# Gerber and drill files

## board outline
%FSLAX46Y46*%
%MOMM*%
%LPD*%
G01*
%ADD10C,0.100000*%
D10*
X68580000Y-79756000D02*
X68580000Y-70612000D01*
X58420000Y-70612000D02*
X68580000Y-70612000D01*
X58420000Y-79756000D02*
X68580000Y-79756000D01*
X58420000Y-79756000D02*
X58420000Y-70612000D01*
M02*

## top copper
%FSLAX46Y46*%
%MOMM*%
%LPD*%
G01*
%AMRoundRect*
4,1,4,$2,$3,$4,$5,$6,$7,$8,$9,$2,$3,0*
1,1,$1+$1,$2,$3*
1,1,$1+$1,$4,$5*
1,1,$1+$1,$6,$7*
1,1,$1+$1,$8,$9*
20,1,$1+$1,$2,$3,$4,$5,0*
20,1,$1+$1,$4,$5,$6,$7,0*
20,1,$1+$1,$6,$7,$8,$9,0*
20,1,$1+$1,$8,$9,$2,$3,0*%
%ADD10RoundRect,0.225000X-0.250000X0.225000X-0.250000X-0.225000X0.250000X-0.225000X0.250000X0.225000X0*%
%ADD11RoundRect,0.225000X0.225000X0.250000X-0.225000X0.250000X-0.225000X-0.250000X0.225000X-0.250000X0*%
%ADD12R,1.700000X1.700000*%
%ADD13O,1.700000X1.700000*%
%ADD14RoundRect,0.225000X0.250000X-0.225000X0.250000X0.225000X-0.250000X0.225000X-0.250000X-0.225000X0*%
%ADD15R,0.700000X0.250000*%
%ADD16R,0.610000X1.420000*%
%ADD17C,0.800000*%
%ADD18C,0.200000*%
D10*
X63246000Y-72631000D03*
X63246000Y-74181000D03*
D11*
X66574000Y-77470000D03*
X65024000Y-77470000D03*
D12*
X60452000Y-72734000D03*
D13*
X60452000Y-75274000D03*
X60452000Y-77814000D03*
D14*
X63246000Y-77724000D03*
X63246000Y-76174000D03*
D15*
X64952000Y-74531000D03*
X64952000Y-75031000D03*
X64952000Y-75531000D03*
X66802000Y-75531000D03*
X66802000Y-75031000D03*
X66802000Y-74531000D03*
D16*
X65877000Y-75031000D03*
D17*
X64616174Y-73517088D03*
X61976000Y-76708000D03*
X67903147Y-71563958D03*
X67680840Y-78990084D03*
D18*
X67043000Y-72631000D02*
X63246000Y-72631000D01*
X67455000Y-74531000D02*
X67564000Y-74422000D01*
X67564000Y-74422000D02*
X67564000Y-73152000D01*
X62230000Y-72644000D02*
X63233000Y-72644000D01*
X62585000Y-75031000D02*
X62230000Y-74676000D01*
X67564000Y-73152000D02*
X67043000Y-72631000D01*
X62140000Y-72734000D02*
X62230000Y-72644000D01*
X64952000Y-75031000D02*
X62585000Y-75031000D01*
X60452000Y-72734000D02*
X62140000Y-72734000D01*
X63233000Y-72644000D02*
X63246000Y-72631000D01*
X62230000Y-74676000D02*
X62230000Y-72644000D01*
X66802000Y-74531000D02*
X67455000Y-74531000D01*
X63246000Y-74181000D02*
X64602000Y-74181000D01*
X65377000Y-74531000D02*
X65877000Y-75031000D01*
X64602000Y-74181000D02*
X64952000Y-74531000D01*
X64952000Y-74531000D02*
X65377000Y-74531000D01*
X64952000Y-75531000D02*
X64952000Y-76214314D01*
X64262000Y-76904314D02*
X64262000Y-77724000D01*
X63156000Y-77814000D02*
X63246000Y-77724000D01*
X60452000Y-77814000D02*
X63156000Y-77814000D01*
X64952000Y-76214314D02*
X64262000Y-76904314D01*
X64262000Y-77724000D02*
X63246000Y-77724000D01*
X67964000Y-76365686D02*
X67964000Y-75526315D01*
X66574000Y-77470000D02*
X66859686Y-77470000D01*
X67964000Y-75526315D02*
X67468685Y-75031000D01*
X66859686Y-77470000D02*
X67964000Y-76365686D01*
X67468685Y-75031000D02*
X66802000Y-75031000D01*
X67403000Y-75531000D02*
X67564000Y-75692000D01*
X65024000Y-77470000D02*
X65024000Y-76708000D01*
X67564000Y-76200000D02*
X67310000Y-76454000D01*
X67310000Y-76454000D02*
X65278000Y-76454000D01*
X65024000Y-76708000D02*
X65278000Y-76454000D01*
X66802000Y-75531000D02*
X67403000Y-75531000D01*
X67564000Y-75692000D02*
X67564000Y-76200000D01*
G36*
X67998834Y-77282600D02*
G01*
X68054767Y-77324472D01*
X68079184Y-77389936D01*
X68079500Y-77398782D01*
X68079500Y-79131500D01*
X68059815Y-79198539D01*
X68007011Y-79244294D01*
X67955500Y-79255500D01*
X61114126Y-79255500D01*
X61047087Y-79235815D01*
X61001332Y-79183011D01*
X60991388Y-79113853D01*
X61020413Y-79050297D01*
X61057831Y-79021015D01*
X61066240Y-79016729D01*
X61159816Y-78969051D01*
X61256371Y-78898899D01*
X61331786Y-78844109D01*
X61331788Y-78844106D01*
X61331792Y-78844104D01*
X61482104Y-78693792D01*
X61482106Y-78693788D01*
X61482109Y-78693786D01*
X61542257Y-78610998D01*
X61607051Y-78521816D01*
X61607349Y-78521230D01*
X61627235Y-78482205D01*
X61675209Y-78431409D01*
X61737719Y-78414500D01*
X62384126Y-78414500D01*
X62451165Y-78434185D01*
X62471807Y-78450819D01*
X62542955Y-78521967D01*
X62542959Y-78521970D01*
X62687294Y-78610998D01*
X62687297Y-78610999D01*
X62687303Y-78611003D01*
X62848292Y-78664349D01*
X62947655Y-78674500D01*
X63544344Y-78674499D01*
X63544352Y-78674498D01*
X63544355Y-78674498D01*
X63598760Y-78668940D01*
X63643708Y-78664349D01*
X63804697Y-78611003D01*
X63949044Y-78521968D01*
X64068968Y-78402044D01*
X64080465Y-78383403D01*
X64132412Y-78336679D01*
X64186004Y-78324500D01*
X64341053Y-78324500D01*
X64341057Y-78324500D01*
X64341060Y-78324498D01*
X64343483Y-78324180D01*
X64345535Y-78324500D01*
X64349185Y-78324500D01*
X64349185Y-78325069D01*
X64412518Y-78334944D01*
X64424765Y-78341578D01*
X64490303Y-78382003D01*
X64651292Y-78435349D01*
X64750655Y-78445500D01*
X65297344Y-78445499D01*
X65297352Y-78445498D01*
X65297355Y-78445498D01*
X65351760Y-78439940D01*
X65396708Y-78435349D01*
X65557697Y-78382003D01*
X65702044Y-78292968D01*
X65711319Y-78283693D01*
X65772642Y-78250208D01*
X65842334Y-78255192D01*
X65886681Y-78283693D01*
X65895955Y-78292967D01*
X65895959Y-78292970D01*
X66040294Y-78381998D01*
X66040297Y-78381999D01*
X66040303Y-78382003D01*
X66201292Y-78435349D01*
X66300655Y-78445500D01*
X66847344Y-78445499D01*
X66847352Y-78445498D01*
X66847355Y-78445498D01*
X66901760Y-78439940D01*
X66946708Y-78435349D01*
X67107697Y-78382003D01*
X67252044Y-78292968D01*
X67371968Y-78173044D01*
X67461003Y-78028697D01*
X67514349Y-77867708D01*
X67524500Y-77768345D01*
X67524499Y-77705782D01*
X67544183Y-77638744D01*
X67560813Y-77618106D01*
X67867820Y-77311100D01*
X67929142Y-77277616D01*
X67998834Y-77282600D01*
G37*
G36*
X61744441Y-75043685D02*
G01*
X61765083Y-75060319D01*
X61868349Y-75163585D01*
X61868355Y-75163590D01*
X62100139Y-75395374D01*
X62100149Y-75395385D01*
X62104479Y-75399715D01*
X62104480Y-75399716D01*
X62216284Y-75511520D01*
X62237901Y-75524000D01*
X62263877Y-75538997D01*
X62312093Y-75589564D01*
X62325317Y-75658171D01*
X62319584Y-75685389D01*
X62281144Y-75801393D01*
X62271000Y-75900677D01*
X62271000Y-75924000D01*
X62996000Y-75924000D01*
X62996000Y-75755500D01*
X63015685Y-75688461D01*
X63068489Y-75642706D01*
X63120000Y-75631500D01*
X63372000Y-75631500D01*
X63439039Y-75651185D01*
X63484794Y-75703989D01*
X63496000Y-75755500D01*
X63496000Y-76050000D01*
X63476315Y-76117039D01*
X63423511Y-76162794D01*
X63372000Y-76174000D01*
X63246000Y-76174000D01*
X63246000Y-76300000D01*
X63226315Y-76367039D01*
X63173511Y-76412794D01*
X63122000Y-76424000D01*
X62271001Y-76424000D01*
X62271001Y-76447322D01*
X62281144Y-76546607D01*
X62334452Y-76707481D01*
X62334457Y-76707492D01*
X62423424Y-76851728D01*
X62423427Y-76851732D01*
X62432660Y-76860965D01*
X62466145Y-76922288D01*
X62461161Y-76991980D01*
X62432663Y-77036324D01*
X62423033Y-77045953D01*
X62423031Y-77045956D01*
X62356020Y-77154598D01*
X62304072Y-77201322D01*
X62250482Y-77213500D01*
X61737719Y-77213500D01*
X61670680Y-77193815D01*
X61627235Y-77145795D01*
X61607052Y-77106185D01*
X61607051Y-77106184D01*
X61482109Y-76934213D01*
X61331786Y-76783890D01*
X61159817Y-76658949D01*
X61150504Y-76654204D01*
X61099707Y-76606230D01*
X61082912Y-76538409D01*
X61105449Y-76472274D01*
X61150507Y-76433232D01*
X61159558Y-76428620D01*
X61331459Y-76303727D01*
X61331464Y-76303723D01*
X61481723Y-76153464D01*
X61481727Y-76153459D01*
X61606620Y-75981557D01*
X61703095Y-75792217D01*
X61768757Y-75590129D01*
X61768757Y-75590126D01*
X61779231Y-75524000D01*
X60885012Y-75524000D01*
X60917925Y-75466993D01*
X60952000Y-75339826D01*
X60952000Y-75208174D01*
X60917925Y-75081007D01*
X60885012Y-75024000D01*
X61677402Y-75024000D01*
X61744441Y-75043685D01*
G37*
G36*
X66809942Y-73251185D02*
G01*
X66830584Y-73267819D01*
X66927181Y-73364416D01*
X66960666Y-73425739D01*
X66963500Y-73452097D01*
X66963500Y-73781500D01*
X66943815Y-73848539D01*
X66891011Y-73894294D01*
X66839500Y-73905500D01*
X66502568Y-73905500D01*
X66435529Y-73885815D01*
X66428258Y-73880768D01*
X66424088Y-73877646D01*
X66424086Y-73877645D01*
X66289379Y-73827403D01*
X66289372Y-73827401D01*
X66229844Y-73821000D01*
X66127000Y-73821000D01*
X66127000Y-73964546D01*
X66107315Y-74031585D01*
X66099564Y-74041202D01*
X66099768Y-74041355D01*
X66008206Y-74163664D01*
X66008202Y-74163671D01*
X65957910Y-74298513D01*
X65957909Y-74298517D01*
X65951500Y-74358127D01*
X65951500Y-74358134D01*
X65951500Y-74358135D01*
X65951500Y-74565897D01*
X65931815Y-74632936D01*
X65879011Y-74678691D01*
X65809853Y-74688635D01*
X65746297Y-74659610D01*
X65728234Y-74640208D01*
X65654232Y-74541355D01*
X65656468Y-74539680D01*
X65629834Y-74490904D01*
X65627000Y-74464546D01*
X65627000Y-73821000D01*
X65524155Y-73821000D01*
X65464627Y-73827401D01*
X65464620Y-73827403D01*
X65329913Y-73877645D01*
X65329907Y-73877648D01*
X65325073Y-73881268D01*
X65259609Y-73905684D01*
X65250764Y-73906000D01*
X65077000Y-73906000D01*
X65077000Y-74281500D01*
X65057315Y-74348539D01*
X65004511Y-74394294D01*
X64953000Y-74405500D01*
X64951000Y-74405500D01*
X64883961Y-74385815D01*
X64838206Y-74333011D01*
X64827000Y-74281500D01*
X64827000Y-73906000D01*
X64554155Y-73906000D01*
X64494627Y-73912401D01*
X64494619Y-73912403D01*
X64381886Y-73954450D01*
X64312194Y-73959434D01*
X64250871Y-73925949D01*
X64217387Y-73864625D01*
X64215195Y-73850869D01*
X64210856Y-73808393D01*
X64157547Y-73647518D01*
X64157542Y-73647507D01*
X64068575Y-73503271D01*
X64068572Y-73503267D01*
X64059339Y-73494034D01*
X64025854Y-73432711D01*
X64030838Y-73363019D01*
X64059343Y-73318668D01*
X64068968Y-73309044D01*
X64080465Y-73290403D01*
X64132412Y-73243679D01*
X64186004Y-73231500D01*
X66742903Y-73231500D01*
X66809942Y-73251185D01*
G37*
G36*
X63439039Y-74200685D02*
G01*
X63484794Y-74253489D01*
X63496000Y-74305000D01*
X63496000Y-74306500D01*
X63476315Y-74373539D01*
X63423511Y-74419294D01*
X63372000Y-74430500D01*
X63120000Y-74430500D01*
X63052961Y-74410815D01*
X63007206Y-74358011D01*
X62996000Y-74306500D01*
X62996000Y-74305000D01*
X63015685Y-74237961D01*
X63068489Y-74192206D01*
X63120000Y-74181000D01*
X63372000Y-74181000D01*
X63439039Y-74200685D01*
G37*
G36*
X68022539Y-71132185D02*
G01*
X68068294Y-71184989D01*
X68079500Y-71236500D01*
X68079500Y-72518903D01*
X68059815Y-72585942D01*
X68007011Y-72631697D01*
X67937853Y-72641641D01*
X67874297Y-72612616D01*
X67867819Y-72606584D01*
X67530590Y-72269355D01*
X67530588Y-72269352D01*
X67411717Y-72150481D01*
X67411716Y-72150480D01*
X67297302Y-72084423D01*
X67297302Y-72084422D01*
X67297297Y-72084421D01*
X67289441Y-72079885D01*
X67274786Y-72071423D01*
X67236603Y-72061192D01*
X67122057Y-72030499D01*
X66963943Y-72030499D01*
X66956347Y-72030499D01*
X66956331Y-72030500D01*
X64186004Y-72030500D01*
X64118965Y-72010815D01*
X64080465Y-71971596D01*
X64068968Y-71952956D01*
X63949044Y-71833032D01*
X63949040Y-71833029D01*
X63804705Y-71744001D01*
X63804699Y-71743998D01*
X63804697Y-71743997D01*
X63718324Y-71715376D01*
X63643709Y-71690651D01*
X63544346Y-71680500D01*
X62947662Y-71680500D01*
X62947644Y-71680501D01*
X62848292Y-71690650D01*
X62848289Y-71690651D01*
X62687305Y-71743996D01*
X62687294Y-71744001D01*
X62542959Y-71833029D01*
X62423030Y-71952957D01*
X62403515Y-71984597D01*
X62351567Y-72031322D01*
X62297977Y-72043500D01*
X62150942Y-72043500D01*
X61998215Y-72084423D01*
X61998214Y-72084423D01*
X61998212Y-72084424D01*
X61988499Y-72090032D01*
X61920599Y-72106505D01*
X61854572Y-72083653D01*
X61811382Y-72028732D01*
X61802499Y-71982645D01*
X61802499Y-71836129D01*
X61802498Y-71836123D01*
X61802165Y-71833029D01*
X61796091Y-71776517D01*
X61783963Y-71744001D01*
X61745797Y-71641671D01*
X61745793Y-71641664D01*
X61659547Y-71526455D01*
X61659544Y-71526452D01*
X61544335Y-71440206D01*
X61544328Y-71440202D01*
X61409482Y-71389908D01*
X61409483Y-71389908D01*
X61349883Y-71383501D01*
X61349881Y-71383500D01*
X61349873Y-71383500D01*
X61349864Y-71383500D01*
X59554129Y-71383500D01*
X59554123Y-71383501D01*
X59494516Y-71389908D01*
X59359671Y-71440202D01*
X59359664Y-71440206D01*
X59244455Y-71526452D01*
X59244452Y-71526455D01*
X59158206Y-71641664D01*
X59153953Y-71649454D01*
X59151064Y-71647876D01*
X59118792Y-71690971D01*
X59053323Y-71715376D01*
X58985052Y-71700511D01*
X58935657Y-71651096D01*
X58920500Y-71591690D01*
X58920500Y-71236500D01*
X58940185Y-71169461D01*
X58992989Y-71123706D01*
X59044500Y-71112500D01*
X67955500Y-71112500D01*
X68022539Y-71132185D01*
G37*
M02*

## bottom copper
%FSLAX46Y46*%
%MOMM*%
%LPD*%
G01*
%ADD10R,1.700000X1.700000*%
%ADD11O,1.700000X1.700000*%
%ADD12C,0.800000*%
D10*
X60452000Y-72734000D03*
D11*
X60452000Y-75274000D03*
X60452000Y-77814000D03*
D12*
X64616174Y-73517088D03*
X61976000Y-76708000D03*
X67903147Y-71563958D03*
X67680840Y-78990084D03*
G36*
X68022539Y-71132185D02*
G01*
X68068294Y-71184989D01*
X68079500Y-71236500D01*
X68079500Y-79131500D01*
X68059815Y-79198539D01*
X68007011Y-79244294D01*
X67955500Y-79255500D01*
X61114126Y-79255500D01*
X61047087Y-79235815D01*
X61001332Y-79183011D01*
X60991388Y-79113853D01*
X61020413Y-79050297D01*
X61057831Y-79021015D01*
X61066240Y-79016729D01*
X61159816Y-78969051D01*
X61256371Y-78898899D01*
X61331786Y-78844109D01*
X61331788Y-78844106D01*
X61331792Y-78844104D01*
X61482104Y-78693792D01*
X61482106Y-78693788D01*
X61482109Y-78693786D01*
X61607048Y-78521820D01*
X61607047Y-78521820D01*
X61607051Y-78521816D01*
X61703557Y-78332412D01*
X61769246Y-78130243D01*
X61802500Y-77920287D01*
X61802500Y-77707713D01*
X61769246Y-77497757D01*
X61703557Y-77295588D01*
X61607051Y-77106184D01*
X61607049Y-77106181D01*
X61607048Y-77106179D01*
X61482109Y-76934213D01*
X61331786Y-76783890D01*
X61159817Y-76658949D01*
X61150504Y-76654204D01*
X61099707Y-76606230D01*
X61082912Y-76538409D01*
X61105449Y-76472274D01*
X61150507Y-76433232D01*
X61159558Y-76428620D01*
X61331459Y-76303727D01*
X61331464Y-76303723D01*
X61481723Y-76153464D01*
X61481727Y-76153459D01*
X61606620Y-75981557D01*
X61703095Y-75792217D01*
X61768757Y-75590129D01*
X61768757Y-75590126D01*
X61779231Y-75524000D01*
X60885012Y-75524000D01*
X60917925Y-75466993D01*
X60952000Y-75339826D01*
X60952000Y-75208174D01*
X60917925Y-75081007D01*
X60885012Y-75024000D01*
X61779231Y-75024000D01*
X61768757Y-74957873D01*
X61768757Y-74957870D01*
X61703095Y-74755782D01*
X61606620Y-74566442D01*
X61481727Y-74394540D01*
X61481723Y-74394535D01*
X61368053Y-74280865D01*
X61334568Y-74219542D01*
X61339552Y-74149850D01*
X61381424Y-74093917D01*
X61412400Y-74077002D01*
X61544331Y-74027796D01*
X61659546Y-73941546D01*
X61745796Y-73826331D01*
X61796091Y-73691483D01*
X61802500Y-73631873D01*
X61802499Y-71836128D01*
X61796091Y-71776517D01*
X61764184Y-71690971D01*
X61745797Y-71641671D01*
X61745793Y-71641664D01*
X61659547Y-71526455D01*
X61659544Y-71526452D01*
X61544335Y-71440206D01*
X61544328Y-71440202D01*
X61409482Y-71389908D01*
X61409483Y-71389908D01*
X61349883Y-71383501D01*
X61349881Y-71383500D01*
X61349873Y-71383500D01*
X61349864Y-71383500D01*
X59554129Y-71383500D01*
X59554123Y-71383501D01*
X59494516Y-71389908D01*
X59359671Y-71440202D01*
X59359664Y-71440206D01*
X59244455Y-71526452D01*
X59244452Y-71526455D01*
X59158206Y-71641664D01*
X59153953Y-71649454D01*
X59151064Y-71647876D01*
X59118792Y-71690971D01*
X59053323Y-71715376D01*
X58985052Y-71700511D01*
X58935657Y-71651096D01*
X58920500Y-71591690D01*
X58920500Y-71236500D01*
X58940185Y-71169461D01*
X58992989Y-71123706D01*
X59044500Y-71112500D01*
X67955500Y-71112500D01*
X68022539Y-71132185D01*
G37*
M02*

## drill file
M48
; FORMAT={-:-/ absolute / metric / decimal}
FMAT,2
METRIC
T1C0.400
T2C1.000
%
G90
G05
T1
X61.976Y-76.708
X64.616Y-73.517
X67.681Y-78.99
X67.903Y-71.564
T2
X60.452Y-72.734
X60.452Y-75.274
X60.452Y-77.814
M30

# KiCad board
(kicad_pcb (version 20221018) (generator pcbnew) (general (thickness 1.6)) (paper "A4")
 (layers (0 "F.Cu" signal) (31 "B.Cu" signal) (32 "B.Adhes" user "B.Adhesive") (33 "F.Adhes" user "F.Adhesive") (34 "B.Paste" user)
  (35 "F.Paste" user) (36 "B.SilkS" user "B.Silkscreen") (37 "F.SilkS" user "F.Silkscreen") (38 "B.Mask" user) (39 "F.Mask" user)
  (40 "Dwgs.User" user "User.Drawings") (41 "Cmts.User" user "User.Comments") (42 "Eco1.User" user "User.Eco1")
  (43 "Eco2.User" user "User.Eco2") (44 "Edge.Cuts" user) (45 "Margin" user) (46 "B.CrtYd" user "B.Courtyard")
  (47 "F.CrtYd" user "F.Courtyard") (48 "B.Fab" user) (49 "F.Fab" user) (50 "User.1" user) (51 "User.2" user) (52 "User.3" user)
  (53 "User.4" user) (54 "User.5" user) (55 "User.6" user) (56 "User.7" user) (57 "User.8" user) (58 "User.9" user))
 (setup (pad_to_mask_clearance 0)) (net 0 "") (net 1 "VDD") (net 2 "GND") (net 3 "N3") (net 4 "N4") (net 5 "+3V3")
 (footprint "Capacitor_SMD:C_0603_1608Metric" (layer "F.Cu") (at 63.246 73.406 -90)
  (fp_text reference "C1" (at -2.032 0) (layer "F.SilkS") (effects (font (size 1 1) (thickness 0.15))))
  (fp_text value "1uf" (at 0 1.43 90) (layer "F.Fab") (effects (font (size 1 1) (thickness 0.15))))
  (pad "1" smd roundrect (at -0.775 0 270) (size 0.9 0.95) (layers "F.Cu" "F.Paste" "F.Mask") (roundrect_rratio 0.25) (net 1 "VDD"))
  (pad "2" smd roundrect (at 0.775 0 270) (size 0.9 0.95) (layers "F.Cu" "F.Paste" "F.Mask") (roundrect_rratio 0.25) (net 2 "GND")))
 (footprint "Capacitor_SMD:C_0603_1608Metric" (layer "F.Cu") (at 65.799 77.47 180)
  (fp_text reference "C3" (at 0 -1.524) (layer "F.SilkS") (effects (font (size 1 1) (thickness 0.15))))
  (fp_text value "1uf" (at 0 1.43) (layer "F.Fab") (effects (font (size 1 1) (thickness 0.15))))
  (pad "1" smd roundrect (at -0.775 0 180) (size 0.9 0.95) (layers "F.Cu" "F.Paste" "F.Mask") (roundrect_rratio 0.25) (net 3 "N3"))
  (pad "2" smd roundrect (at 0.775 0 180) (size 0.9 0.95) (layers "F.Cu" "F.Paste" "F.Mask") (roundrect_rratio 0.25) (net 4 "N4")))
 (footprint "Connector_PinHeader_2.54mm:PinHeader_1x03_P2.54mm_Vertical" (layer "F.Cu") (at 60.452 72.734)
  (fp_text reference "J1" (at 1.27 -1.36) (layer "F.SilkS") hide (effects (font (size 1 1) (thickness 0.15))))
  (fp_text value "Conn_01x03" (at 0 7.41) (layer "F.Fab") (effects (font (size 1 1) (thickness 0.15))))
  (pad "1" thru_hole rect (at 0 0) (size 1.7 1.7) (drill 1) (layers "*.Cu" "*.Mask") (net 1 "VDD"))
  (pad "2" thru_hole oval (at 0 2.54) (size 1.7 1.7) (drill 1) (layers "*.Cu" "*.Mask") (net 2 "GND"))
  (pad "3" thru_hole oval (at 0 5.08) (size 1.7 1.7) (drill 1) (layers "*.Cu" "*.Mask") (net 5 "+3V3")))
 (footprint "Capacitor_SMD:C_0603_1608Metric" (layer "F.Cu") (at 63.246 76.949 90)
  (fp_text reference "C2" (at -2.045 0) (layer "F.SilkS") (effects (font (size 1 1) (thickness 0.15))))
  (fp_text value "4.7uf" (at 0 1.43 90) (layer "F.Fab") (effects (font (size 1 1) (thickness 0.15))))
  (pad "1" smd roundrect (at -0.775 0 90) (size 0.9 0.95) (layers "F.Cu" "F.Paste" "F.Mask") (roundrect_rratio 0.25) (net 5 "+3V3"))
  (pad "2" smd roundrect (at 0.775 0 90) (size 0.9 0.95) (layers "F.Cu" "F.Paste" "F.Mask") (roundrect_rratio 0.25) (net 2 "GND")))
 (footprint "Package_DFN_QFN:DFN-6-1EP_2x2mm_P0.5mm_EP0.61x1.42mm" (layer "F.Cu") (at 65.877 75.031)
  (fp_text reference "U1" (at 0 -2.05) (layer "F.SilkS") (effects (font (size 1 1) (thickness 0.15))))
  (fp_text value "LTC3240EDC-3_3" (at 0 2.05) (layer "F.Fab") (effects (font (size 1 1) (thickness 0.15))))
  (pad "" smd rect (at 0 -0.355) (size 0.5 0.56) (layers "F.Paste"))
  (pad "" smd rect (at 0 0.355) (size 0.5 0.56) (layers "F.Paste"))
  (pad "1" smd rect (at -0.925 -0.5) (size 0.7 0.25) (layers "F.Cu" "F.Paste" "F.Mask") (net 2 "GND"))
  (pad "2" smd rect (at -0.925 0) (size 0.7 0.25) (layers "F.Cu" "F.Paste" "F.Mask") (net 1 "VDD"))
  (pad "3" smd rect (at -0.925 0.5) (size 0.7 0.25) (layers "F.Cu" "F.Paste" "F.Mask") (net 5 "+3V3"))
  (pad "4" smd rect (at 0.925 0.5) (size 0.7 0.25) (layers "F.Cu" "F.Paste" "F.Mask") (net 4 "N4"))
  (pad "5" smd rect (at 0.925 0) (size 0.7 0.25) (layers "F.Cu" "F.Paste" "F.Mask") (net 3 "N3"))
  (pad "6" smd rect (at 0.925 -0.5) (size 0.7 0.25) (layers "F.Cu" "F.Paste" "F.Mask") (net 1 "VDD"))
  (pad "7" smd rect (at 0 0) (size 0.61 1.42) (layers "F.Cu" "F.Mask") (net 2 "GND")))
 (gr_line (start 68.58 79.756) (end 68.58 70.612) (stroke (width 0.1) (type default)) (layer "Edge.Cuts"))
 (gr_line (start 58.42 70.612) (end 68.58 70.612) (stroke (width 0.1) (type default)) (layer "Edge.Cuts"))
 (gr_line (start 58.42 79.756) (end 68.58 79.756) (stroke (width 0.1) (type default)) (layer "Edge.Cuts"))
 (gr_line (start 58.42 79.756) (end 58.42 70.612) (stroke (width 0.1) (type default)) (layer "Edge.Cuts"))
 (segment (start 67.043 72.631) (end 63.246 72.631) (width 0.2) (layer "F.Cu") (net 1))
 (segment (start 67.455 74.531) (end 67.564 74.422) (width 0.2) (layer "F.Cu") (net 1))
 (segment (start 67.564 74.422) (end 67.564 73.152) (width 0.2) (layer "F.Cu") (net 1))
 (segment (start 62.23 72.644) (end 63.233 72.644) (width 0.2) (layer "F.Cu") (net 1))
 (segment (start 62.585 75.031) (end 62.23 74.676) (width 0.2) (layer "F.Cu") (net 1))
 (segment (start 67.564 73.152) (end 67.043 72.631) (width 0.2) (layer "F.Cu") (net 1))
 (segment (start 62.14 72.734) (end 62.23 72.644) (width 0.2) (layer "F.Cu") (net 1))
 (segment (start 64.952 75.031) (end 62.585 75.031) (width 0.2) (layer "F.Cu") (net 1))
 (segment (start 60.452 72.734) (end 62.14 72.734) (width 0.2) (layer "F.Cu") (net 1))
 (segment (start 63.233 72.644) (end 63.246 72.631) (width 0.2) (layer "F.Cu") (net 1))
 (segment (start 62.23 74.676) (end 62.23 72.644) (width 0.2) (layer "F.Cu") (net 1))
 (segment (start 66.802 74.531) (end 67.455 74.531) (width 0.2) (layer "F.Cu") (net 1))
 (segment (start 63.246 74.181) (end 64.602 74.181) (width 0.2) (layer "F.Cu") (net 2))
 (segment (start 65.377 74.531) (end 65.877 75.031) (width 0.2) (layer "F.Cu") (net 2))
 (segment (start 64.602 74.181) (end 64.952 74.531) (width 0.2) (layer "F.Cu") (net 2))
 (segment (start 64.952 74.531) (end 65.377 74.531) (width 0.2) (layer "F.Cu") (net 2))
 (via (at 64.616174 73.517088) (size 0.8) (drill 0.4) (layers "F.Cu" "B.Cu") (free) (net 2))
 (via (at 61.976 76.708) (size 0.8) (drill 0.4) (layers "F.Cu" "B.Cu") (free) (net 2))
 (via (at 67.903147 71.563958) (size 0.8) (drill 0.4) (layers "F.Cu" "B.Cu") (free) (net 2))
 (via (at 67.68084 78.990084) (size 0.8) (drill 0.4) (layers "F.Cu" "B.Cu") (free) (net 2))
 (segment (start 64.952 75.531) (end 64.952 76.214314) (width 0.2) (layer "F.Cu") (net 5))
 (segment (start 64.262 76.904314) (end 64.262 77.724) (width 0.2) (layer "F.Cu") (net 5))
 (segment (start 63.156 77.814) (end 63.246 77.724) (width 0.2) (layer "F.Cu") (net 5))
 (segment (start 60.452 77.814) (end 63.156 77.814) (width 0.2) (layer "F.Cu") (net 5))
 (segment (start 64.952 76.214314) (end 64.262 76.904314) (width 0.2) (layer "F.Cu") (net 5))
 (segment (start 64.262 77.724) (end 63.246 77.724) (width 0.2) (layer "F.Cu") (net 5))
 (segment (start 67.964 76.365686) (end 67.964 75.526315) (width 0.2) (layer "F.Cu") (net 3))
 (segment (start 66.574 77.47) (end 66.859686 77.47) (width 0.2) (layer "F.Cu") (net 3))
 (segment (start 67.964 75.526315) (end 67.468685 75.031) (width 0.2) (layer "F.Cu") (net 3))
 (segment (start 66.859686 77.47) (end 67.964 76.365686) (width 0.2) (layer "F.Cu") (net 3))
 (segment (start 67.468685 75.031) (end 66.802 75.031) (width 0.2) (layer "F.Cu") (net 3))
 (segment (start 67.403 75.531) (end 67.564 75.692) (width 0.2) (layer "F.Cu") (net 4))
 (segment (start 65.024 77.47) (end 65.024 76.708) (width 0.2) (layer "F.Cu") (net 4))
 (segment (start 67.564 76.2) (end 67.31 76.454) (width 0.2) (layer "F.Cu") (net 4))
 (segment (start 67.31 76.454) (end 65.278 76.454) (width 0.2) (layer "F.Cu") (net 4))
 (segment (start 65.024 76.708) (end 65.278 76.454) (width 0.2) (layer "F.Cu") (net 4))
 (segment (start 66.802 75.531) (end 67.403 75.531) (width 0.2) (layer "F.Cu") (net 4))
 (segment (start 67.564 75.692) (end 67.564 76.2) (width 0.2) (layer "F.Cu") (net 4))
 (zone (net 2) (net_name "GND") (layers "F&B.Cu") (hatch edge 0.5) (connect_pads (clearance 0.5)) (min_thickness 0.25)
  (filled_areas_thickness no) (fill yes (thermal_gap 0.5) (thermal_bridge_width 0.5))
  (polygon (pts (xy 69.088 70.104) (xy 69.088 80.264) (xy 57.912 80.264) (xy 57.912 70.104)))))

